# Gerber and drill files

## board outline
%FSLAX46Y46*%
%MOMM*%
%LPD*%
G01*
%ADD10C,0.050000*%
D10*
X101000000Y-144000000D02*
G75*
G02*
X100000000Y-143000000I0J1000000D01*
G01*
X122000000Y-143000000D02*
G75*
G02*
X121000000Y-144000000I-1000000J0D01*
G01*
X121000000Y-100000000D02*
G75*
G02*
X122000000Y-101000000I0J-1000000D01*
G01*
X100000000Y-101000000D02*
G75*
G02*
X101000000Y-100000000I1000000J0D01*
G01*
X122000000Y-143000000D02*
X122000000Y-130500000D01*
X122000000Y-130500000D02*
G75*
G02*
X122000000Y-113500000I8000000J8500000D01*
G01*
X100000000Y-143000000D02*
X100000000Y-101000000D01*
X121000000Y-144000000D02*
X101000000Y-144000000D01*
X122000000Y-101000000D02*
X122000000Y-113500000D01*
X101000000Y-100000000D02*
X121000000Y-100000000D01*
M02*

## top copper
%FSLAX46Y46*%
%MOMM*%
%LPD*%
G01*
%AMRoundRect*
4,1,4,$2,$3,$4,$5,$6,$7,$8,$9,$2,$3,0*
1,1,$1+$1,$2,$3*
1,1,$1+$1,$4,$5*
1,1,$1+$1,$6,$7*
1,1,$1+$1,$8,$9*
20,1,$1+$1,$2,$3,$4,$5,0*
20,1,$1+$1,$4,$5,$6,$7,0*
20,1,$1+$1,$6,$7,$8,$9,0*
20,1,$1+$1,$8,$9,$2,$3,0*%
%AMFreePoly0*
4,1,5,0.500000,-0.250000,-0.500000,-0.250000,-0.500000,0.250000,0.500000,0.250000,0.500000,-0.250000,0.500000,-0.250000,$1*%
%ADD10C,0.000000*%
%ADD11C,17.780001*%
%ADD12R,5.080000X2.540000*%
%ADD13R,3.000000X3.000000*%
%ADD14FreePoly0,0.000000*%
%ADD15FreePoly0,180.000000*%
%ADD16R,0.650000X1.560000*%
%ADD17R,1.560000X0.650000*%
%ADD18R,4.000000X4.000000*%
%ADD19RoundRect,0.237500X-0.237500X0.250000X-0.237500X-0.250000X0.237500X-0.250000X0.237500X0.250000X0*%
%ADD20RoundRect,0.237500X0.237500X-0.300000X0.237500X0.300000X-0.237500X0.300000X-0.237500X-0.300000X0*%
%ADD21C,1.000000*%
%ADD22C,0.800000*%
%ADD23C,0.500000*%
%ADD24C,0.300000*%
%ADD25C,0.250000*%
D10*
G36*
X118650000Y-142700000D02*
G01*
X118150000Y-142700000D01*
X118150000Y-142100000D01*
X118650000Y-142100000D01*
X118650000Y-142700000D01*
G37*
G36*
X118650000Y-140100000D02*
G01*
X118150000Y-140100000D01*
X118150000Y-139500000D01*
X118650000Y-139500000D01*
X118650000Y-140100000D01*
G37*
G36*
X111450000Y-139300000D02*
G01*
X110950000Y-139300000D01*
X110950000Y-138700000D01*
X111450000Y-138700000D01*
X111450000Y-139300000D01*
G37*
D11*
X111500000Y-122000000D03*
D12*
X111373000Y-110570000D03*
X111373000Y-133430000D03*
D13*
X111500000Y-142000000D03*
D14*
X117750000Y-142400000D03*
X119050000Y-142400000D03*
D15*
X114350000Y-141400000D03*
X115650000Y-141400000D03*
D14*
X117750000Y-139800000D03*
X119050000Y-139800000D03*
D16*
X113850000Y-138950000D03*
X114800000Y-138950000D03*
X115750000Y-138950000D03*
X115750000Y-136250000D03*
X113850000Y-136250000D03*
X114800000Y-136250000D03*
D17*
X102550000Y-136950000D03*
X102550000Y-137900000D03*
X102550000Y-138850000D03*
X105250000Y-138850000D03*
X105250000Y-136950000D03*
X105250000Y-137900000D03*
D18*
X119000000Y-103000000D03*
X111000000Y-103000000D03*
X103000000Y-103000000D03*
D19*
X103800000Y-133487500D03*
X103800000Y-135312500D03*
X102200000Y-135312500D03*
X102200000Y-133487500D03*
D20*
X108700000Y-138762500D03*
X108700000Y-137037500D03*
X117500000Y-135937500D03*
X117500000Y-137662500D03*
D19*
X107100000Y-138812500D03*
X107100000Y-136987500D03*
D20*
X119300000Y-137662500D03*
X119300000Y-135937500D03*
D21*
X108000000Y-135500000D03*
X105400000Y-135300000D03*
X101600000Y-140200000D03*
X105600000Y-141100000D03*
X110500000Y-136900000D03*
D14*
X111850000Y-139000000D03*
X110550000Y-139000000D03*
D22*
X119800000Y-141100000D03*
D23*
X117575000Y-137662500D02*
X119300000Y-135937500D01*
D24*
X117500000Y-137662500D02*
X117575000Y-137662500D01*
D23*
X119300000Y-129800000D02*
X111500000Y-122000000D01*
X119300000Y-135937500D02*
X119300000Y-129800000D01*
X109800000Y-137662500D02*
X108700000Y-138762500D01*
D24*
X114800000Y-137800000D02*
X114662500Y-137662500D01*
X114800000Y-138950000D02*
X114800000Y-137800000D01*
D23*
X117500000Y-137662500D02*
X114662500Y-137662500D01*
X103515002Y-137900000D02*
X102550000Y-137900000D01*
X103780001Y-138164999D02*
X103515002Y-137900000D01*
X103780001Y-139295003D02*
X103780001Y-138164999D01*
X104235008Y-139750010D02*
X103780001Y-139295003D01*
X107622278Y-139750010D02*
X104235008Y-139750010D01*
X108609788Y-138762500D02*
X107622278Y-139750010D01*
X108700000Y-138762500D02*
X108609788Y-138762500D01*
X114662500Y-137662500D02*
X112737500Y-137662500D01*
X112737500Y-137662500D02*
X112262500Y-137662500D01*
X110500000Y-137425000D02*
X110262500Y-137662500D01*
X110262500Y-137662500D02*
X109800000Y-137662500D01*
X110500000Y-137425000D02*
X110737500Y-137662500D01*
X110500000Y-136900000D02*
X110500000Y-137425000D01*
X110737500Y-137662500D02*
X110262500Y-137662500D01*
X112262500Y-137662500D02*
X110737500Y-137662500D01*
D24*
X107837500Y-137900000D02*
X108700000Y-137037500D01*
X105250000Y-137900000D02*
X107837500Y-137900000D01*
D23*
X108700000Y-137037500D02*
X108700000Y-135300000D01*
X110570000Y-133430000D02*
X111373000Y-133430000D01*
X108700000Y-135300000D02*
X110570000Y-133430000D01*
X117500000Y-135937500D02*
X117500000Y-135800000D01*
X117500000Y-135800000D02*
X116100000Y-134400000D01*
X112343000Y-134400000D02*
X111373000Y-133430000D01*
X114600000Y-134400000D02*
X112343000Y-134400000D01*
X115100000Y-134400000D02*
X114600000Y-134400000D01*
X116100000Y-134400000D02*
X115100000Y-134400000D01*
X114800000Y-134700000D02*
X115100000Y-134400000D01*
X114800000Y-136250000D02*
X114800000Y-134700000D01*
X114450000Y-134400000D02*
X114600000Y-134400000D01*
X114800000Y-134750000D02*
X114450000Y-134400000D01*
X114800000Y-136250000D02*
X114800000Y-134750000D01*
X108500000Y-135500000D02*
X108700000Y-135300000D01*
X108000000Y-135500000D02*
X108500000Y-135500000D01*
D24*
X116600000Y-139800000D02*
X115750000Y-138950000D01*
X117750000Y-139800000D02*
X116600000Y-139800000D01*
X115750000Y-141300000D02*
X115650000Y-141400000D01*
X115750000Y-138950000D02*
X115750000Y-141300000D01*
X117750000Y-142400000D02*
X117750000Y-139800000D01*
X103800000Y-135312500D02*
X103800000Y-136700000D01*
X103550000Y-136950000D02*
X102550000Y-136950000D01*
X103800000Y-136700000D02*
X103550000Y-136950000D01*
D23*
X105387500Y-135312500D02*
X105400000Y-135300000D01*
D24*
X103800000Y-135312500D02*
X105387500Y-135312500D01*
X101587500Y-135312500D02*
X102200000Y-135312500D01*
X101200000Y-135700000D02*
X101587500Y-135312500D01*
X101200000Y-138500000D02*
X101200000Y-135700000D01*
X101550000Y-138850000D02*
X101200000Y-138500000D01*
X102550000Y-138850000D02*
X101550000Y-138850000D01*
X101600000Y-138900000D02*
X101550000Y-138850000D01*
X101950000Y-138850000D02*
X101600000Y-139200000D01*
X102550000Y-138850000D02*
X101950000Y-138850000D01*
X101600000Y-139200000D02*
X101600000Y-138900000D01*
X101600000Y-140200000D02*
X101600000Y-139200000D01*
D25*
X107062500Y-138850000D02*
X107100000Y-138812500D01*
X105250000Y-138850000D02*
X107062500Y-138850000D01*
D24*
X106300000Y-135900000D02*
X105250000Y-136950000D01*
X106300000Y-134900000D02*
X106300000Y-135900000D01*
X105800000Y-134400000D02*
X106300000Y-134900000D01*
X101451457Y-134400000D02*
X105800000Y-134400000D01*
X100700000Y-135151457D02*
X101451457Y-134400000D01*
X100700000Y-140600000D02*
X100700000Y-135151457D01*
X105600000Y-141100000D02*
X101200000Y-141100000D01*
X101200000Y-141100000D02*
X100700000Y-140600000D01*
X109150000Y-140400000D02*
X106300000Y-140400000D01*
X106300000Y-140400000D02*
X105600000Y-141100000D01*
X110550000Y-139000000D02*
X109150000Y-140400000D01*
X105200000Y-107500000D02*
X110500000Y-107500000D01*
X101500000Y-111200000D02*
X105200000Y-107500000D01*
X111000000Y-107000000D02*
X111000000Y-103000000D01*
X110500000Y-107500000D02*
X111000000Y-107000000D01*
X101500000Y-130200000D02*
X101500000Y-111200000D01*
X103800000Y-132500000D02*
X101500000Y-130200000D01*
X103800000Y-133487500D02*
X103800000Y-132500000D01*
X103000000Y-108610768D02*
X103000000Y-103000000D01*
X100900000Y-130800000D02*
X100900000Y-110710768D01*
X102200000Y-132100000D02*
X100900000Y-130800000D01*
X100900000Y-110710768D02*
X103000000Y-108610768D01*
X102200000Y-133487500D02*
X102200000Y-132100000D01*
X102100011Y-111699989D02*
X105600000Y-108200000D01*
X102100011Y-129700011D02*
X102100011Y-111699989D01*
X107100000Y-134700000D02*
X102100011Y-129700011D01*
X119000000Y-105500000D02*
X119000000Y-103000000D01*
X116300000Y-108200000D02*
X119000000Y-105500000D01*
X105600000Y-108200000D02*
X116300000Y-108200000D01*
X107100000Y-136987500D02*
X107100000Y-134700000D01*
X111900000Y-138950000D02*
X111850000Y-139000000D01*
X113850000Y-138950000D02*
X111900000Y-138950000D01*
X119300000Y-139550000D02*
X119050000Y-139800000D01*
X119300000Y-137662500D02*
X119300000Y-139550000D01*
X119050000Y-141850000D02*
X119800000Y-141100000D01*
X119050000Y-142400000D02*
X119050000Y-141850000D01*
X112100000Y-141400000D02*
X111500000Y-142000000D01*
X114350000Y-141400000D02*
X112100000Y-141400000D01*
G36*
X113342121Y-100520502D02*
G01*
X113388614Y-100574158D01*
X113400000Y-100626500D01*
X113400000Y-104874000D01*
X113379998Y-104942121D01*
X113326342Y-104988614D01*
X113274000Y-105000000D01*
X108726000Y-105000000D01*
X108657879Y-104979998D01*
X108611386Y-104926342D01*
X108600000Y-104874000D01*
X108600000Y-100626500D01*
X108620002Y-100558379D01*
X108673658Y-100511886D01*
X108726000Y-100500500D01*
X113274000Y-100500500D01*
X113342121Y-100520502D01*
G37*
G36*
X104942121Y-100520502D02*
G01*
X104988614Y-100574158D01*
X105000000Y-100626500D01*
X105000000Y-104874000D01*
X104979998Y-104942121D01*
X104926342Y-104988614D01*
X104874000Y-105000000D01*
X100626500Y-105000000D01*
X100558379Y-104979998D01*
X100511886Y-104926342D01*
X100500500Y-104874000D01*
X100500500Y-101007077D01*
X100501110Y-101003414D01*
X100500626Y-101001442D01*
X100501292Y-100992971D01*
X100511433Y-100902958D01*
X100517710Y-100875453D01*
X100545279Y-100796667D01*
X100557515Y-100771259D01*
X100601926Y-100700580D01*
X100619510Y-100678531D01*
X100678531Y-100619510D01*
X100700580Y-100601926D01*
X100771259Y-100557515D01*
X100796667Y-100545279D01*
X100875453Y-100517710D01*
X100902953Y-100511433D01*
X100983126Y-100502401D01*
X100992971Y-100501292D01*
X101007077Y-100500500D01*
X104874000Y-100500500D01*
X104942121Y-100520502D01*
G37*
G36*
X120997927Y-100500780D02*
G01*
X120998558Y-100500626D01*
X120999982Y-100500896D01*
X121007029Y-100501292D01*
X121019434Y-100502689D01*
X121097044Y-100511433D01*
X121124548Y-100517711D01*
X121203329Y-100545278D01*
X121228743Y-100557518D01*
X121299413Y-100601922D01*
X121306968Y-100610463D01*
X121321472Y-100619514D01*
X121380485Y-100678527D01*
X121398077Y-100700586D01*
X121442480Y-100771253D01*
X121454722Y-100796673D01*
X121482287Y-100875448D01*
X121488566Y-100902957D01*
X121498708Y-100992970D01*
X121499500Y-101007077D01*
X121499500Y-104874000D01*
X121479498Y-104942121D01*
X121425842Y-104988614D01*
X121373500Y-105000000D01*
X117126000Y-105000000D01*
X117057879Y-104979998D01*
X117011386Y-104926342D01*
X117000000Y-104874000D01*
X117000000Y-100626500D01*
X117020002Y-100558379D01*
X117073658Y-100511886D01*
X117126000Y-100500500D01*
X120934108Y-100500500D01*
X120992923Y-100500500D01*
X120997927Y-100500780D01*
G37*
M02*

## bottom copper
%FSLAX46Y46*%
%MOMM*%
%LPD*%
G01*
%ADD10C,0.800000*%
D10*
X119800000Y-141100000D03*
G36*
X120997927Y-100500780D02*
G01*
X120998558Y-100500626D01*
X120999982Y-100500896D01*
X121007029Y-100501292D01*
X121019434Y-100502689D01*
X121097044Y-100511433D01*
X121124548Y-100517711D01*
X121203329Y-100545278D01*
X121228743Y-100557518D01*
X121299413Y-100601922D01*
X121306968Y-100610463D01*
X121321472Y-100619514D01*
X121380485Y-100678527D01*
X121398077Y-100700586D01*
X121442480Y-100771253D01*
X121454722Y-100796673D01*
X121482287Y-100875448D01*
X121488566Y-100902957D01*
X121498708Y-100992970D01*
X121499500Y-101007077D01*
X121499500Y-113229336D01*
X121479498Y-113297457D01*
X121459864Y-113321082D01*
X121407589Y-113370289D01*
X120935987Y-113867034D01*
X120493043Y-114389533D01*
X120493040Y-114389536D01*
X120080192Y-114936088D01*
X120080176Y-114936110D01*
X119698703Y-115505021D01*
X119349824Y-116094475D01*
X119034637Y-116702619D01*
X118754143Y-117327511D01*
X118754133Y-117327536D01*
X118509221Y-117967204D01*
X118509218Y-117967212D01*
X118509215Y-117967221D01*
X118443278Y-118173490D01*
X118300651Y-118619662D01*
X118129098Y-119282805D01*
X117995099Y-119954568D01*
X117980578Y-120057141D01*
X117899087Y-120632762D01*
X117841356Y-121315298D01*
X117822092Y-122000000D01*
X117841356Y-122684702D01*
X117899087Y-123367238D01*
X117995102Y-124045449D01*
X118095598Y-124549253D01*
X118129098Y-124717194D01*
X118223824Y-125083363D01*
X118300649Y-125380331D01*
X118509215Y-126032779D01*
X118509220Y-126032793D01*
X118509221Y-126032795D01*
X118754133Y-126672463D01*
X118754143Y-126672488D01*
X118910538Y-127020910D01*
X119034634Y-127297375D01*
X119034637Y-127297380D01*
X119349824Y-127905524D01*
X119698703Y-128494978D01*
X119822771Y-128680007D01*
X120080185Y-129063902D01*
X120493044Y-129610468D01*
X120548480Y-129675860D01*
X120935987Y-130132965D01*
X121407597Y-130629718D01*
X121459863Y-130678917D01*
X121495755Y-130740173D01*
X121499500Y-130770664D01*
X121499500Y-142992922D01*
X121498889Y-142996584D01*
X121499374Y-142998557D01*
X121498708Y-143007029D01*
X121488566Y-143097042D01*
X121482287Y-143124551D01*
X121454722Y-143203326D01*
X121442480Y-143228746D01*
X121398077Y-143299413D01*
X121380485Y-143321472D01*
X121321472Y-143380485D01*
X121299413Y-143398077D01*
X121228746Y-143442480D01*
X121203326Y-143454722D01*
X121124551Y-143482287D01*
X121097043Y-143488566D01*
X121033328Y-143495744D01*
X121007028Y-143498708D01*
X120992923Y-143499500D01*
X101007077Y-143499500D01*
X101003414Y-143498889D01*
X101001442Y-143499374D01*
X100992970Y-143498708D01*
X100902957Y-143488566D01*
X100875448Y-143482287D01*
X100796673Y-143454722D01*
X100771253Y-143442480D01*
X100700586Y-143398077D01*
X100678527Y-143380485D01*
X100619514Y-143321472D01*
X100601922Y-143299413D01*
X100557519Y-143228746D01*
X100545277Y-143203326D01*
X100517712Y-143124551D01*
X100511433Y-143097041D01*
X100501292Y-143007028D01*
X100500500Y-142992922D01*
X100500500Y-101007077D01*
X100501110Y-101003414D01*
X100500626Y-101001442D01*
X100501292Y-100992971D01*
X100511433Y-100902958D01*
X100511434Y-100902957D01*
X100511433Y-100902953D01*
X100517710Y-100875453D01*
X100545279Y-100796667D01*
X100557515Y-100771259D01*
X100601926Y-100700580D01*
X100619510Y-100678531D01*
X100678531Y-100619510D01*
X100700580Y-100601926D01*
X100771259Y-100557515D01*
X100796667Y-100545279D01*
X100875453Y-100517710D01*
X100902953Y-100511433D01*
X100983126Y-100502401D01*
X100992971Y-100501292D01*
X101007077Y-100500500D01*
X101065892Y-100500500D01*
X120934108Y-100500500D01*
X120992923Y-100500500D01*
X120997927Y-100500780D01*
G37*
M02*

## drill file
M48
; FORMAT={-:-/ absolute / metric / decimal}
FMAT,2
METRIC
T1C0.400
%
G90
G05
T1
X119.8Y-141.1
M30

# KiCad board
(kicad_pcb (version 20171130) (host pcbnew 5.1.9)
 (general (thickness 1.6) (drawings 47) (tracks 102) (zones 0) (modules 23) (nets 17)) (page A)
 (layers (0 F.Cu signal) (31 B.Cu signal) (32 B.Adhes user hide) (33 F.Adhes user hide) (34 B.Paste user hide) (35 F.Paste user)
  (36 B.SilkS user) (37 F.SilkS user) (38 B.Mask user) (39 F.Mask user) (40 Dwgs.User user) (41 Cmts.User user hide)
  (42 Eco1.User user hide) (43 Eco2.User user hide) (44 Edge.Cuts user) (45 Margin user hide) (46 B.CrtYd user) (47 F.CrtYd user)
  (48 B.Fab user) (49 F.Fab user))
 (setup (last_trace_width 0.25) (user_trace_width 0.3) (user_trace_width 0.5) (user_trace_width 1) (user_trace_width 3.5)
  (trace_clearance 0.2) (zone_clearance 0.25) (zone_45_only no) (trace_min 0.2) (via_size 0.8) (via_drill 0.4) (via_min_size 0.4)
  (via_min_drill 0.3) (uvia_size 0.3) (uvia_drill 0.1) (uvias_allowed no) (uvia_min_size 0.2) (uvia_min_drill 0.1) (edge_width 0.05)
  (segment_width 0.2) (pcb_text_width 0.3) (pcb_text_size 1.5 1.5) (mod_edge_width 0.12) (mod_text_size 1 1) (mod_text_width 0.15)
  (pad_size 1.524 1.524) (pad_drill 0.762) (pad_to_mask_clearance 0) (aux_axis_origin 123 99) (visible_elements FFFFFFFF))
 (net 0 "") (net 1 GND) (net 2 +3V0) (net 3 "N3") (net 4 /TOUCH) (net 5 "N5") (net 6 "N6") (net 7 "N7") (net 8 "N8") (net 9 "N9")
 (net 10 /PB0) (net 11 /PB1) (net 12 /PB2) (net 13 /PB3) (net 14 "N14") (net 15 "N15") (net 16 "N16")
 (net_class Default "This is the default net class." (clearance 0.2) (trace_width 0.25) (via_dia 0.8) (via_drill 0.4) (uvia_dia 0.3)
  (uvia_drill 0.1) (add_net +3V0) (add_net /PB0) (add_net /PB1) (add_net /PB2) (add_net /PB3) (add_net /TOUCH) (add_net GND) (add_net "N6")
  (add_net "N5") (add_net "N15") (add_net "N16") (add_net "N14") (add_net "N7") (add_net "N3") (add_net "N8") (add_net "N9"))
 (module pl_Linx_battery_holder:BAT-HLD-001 (layer F.Cu) (at 111.5 122 90)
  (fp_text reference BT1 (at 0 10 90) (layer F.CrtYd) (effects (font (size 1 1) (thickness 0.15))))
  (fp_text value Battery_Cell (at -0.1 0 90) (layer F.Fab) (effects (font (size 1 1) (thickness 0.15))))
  (pad 2 smd circle (at 0 0 90) (size 17.780001 17.780001) (layers F.Cu F.Mask) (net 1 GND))
  (pad 3 smd rect (at 11.43 -0.127 90) (size 2.54 5.08) (layers F.Cu F.Paste F.Mask))
  (pad 1 smd rect (at -11.43 -0.127 90) (size 2.54 5.08) (layers F.Cu F.Paste F.Mask) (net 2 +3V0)))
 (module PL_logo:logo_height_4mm (layer F.Cu) (at 118.5 111.5)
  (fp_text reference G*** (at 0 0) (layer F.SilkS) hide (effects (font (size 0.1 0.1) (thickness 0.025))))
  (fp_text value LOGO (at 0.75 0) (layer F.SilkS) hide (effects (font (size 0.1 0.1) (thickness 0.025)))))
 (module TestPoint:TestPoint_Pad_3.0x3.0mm (layer F.Cu) (at 111.5 142)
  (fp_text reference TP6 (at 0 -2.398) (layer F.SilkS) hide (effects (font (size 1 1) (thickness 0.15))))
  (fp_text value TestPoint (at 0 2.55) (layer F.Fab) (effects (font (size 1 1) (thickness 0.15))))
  (pad 1 smd rect (at 0 0) (size 3 3) (layers F.Cu F.Mask) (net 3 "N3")))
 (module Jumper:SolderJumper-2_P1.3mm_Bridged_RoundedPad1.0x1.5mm (layer F.Cu) (at 118.4 142.4)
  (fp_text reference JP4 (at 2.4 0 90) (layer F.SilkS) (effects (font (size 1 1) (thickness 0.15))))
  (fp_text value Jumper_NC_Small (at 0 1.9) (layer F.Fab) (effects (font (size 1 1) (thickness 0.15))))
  (fp_poly (pts (xy 0.25 -0.3) (xy -0.25 -0.3) (xy -0.25 0.3) (xy 0.25 0.3)) (layer F.Cu) (width 0))
  (pad 1 smd custom (at -0.65 0) (size 1 0.5) (layers F.Cu F.Mask) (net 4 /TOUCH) (zone_connect 2)
   (options (clearance outline) (anchor rect)) (primitives))
  (pad 2 smd custom (at 0.65 0) (size 1 0.5) (layers F.Cu F.Mask) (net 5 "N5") (zone_connect 2) (options (clearance outline) (anchor rect))
   (primitives)))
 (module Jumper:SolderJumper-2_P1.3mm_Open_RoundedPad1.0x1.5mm (layer F.Cu) (at 115 141.4 180)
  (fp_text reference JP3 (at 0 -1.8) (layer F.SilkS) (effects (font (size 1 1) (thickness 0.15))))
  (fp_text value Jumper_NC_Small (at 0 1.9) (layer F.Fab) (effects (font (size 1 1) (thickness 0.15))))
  (pad 2 smd custom (at 0.65 0 180) (size 1 0.5) (layers F.Cu F.Mask) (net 3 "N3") (zone_connect 2)
   (options (clearance outline) (anchor rect)) (primitives))
  (pad 1 smd custom (at -0.65 0 180) (size 1 0.5) (layers F.Cu F.Mask) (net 4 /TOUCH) (zone_connect 2)
   (options (clearance outline) (anchor rect)) (primitives)))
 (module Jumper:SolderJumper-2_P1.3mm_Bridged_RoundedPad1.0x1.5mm (layer F.Cu) (at 118.4 139.8)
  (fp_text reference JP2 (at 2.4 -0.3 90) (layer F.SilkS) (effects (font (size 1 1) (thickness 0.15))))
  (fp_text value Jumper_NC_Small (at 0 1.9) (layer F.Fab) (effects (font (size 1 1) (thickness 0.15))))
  (fp_poly (pts (xy 0.25 -0.3) (xy -0.25 -0.3) (xy -0.25 0.3) (xy 0.25 0.3)) (layer F.Cu) (width 0))
  (pad 1 smd custom (at -0.65 0) (size 1 0.5) (layers F.Cu F.Mask) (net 4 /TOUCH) (zone_connect 2)
   (options (clearance outline) (anchor rect)) (primitives))
  (pad 2 smd custom (at 0.65 0) (size 1 0.5) (layers F.Cu F.Mask) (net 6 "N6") (zone_connect 2) (options (clearance outline) (anchor rect))
   (primitives)))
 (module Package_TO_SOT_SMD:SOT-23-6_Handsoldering (layer F.Cu) (at 114.8 137.6 90)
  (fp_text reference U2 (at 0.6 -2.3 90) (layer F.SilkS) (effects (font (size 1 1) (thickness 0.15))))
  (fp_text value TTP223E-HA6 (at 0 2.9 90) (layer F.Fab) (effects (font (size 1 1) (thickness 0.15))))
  (pad 1 smd rect (at -1.35 -0.95 90) (size 1.56 0.65) (layers F.Cu F.Paste F.Mask) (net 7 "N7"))
  (pad 2 smd rect (at -1.35 0 90) (size 1.56 0.65) (layers F.Cu F.Paste F.Mask) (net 1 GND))
  (pad 3 smd rect (at -1.35 0.95 90) (size 1.56 0.65) (layers F.Cu F.Paste F.Mask) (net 4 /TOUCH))
  (pad 4 smd rect (at 1.35 0.95 90) (size 1.56 0.65) (layers F.Cu F.Paste F.Mask) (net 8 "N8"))
  (pad 6 smd rect (at 1.35 -0.95 90) (size 1.56 0.65) (layers F.Cu F.Paste F.Mask) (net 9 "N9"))
  (pad 5 smd rect (at 1.35 0 90) (size 1.56 0.65) (layers F.Cu F.Paste F.Mask) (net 2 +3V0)))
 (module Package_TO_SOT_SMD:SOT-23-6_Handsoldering (layer F.Cu) (at 103.9 137.9)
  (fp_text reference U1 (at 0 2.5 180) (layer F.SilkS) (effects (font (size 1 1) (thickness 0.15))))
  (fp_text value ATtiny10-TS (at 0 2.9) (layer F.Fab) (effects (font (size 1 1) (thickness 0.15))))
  (pad 1 smd rect (at -1.35 -0.95) (size 1.56 0.65) (layers F.Cu F.Paste F.Mask) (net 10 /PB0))
  (pad 2 smd rect (at -1.35 0) (size 1.56 0.65) (layers F.Cu F.Paste F.Mask) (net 1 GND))
  (pad 3 smd rect (at -1.35 0.95) (size 1.56 0.65) (layers F.Cu F.Paste F.Mask) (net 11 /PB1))
  (pad 4 smd rect (at 1.35 0.95) (size 1.56 0.65) (layers F.Cu F.Paste F.Mask) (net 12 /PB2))
  (pad 6 smd rect (at 1.35 -0.95) (size 1.56 0.65) (layers F.Cu F.Paste F.Mask) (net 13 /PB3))
  (pad 5 smd rect (at 1.35 0) (size 1.56 0.65) (layers F.Cu F.Paste F.Mask) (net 2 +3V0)))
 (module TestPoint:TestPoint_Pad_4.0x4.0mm (layer F.Cu) (at 119 103)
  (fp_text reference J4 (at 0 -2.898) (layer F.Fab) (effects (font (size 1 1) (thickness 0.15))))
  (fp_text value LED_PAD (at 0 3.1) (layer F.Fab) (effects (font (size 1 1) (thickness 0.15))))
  (pad 1 smd rect (at 0 0) (size 4 4) (layers F.Cu F.Mask) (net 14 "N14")))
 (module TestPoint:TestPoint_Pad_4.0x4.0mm (layer F.Cu) (at 111 103)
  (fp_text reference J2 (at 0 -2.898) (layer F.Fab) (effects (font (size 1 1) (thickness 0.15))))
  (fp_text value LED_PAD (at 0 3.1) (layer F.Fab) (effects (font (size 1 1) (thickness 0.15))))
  (pad 1 smd rect (at 0 0) (size 4 4) (layers F.Cu F.Mask) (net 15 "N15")))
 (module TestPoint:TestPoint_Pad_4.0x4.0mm (layer F.Cu) (at 103 103)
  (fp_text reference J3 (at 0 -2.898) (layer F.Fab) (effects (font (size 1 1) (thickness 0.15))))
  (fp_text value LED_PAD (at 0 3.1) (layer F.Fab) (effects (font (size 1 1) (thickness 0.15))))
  (pad 1 smd rect (at 0 0) (size 4 4) (layers F.Cu F.Mask) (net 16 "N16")))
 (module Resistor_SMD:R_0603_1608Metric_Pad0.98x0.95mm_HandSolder (layer F.Cu) (at 103.8 134.4 270)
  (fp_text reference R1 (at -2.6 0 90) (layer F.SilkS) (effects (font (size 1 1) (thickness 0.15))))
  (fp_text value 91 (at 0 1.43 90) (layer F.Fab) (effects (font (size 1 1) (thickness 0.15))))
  (pad 1 smd roundrect (at -0.9125 0 270) (size 0.975 0.95) (layers F.Cu F.Paste F.Mask) (roundrect_rratio 0.25) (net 15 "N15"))
  (pad 2 smd roundrect (at 0.9125 0 270) (size 0.975 0.95) (layers F.Cu F.Paste F.Mask) (roundrect_rratio 0.25) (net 10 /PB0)))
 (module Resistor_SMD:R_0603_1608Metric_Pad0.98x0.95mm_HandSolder (layer F.Cu) (at 102.2 134.4 270)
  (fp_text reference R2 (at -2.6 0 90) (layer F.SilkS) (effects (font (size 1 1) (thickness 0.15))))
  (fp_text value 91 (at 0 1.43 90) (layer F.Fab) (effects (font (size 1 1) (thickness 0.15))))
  (pad 2 smd roundrect (at 0.9125 0 270) (size 0.975 0.95) (layers F.Cu F.Paste F.Mask) (roundrect_rratio 0.25) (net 11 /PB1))
  (pad 1 smd roundrect (at -0.9125 0 270) (size 0.975 0.95) (layers F.Cu F.Paste F.Mask) (roundrect_rratio 0.25) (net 16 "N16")))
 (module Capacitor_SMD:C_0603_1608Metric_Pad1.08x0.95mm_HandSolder (layer F.Cu) (at 108.7 137.9 90)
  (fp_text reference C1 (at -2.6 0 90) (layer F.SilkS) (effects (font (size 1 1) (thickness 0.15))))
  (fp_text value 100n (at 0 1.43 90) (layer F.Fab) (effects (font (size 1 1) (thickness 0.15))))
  (pad 1 smd roundrect (at -0.8625 0 90) (size 1.075 0.95) (layers F.Cu F.Paste F.Mask) (roundrect_rratio 0.25) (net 1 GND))
  (pad 2 smd roundrect (at 0.8625 0 90) (size 1.075 0.95) (layers F.Cu F.Paste F.Mask) (roundrect_rratio 0.25) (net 2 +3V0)))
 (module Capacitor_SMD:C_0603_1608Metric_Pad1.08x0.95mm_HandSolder (layer F.Cu) (at 117.5 136.8 90)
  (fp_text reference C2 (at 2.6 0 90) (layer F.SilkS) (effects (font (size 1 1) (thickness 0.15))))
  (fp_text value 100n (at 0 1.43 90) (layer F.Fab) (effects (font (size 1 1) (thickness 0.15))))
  (pad 2 smd roundrect (at 0.8625 0 90) (size 1.075 0.95) (layers F.Cu F.Paste F.Mask) (roundrect_rratio 0.25) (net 2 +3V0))
  (pad 1 smd roundrect (at -0.8625 0 90) (size 1.075 0.95) (layers F.Cu F.Paste F.Mask) (roundrect_rratio 0.25) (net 1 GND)))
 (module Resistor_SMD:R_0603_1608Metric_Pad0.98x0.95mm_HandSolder (layer F.Cu) (at 107.1 137.9 270)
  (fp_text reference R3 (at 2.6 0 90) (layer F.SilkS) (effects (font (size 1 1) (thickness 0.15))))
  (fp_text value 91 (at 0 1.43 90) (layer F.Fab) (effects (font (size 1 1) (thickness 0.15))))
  (pad 2 smd roundrect (at 0.9125 0 270) (size 0.975 0.95) (layers F.Cu F.Paste F.Mask) (roundrect_rratio 0.25) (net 12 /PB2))
  (pad 1 smd roundrect (at -0.9125 0 270) (size 0.975 0.95) (layers F.Cu F.Paste F.Mask) (roundrect_rratio 0.25) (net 14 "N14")))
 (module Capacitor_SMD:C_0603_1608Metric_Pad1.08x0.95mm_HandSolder (layer F.Cu) (at 119.3 136.8 90)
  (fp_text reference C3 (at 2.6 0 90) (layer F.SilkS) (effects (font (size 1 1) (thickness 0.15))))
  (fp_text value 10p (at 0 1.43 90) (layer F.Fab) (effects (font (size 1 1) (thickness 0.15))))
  (pad 1 smd roundrect (at -0.8625 0 90) (size 1.075 0.95) (layers F.Cu F.Paste F.Mask) (roundrect_rratio 0.25) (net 6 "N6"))
  (pad 2 smd roundrect (at 0.8625 0 90) (size 1.075 0.95) (layers F.Cu F.Paste F.Mask) (roundrect_rratio 0.25) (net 1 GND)))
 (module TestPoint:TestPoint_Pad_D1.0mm (layer F.Cu) (at 108 135.5)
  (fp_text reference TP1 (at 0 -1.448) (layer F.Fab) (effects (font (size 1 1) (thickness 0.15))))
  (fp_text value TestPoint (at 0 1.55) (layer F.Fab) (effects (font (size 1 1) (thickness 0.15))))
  (pad 1 smd circle (at 0 0) (size 1 1) (layers F.Cu F.Mask) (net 2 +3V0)))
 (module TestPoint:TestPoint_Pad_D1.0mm (layer F.Cu) (at 105.4 135.3)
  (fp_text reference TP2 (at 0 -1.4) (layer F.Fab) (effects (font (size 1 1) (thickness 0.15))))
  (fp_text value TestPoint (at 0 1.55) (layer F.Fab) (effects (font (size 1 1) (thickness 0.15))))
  (pad 1 smd circle (at 0 0) (size 1 1) (layers F.Cu F.Mask) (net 10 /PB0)))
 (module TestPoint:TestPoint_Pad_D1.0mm (layer F.Cu) (at 101.6 140.2)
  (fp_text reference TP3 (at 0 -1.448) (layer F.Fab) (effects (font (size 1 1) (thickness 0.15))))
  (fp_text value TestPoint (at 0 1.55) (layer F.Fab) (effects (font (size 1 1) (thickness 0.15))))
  (pad 1 smd circle (at 0 0) (size 1 1) (layers F.Cu F.Mask) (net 11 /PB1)))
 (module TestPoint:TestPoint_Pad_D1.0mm (layer F.Cu) (at 105.6 141.1)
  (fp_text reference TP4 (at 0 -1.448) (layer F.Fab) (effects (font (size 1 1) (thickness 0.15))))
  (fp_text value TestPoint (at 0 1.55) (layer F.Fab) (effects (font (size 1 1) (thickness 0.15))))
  (pad 1 smd circle (at 0 0) (size 1 1) (layers F.Cu F.Mask) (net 13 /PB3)))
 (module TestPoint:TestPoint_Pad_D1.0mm (layer F.Cu) (at 110.5 136.9)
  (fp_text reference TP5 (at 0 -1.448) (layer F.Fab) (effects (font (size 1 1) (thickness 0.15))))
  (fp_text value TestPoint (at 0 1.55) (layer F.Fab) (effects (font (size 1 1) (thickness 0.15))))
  (pad 1 smd circle (at 0 0) (size 1 1) (layers F.Cu F.Mask) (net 1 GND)))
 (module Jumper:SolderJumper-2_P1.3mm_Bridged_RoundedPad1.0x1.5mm (layer F.Cu) (at 111.2 139)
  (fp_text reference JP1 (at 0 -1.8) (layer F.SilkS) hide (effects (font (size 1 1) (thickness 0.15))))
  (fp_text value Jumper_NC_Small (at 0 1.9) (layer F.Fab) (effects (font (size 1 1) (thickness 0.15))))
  (fp_poly (pts (xy 0.25 -0.3) (xy -0.25 -0.3) (xy -0.25 0.3) (xy 0.25 0.3)) (layer F.Cu) (width 0))
  (pad 2 smd custom (at 0.65 0) (size 1 0.5) (layers F.Cu F.Mask) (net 7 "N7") (zone_connect 2) (options (clearance outline) (anchor rect))
   (primitives))
  (pad 1 smd custom (at -0.65 0) (size 1 0.5) (layers F.Cu F.Mask) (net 13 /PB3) (zone_connect 2)
   (options (clearance outline) (anchor rect)) (primitives)))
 (gr_arc (start 101 143) (end 100 143) (angle -90) (layer Edge.Cuts) (width 0.05))
 (gr_arc (start 121 143) (end 121 144) (angle -90) (layer Edge.Cuts) (width 0.05))
 (gr_arc (start 121 101) (end 122 101) (angle -90) (layer Edge.Cuts) (width 0.05))
 (gr_arc (start 101 101) (end 101 100) (angle -90) (layer Edge.Cuts) (width 0.05))
 (gr_line (start 122 143) (end 122 130.5) (layer Edge.Cuts) (width 0.05))
 (gr_arc (start 130 122) (end 122 113.5) (angle -93.47140918) (layer Edge.Cuts) (width 0.05))
 (gr_line (start 100 143) (end 100 101) (layer Edge.Cuts) (width 0.05))
 (gr_line (start 121 144) (end 101 144) (layer Edge.Cuts) (width 0.05))
 (gr_line (start 122 101) (end 122 113.5) (layer Edge.Cuts) (width 0.05))
 (gr_line (start 101 100) (end 121 100) (layer Edge.Cuts) (width 0.05))
 (segment (start 117.575 137.6625) (end 119.3 135.9375) (width 0.5) (layer F.Cu) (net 1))
 (segment (start 117.5 137.6625) (end 117.575 137.6625) (width 0.3) (layer F.Cu) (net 1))
 (segment (start 119.3 129.8) (end 111.5 122) (width 0.5) (layer F.Cu) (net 1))
 (segment (start 119.3 135.9375) (end 119.3 129.8) (width 0.5) (layer F.Cu) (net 1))
 (segment (start 109.8 137.6625) (end 108.7 138.7625) (width 0.5) (layer F.Cu) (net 1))
 (segment (start 114.8 137.8) (end 114.6625 137.6625) (width 0.3) (layer F.Cu) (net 1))
 (segment (start 114.8 138.95) (end 114.8 137.8) (width 0.3) (layer F.Cu) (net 1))
 (segment (start 117.5 137.6625) (end 114.6625 137.6625) (width 0.5) (layer F.Cu) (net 1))
 (segment (start 103.515002 137.9) (end 102.55 137.9) (width 0.5) (layer F.Cu) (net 1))
 (segment (start 103.780001 138.164999) (end 103.515002 137.9) (width 0.5) (layer F.Cu) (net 1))
 (segment (start 103.780001 139.295003) (end 103.780001 138.164999) (width 0.5) (layer F.Cu) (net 1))
 (segment (start 104.235008 139.75001) (end 103.780001 139.295003) (width 0.5) (layer F.Cu) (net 1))
 (segment (start 107.622278 139.75001) (end 104.235008 139.75001) (width 0.5) (layer F.Cu) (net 1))
 (segment (start 108.609788 138.7625) (end 107.622278 139.75001) (width 0.5) (layer F.Cu) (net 1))
 (segment (start 108.7 138.7625) (end 108.609788 138.7625) (width 0.5) (layer F.Cu) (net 1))
 (segment (start 114.6625 137.6625) (end 112.7375 137.6625) (width 0.5) (layer F.Cu) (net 1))
 (segment (start 112.7375 137.6625) (end 112.2625 137.6625) (width 0.5) (layer F.Cu) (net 1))
 (segment (start 110.5 137.425) (end 110.2625 137.6625) (width 0.5) (layer F.Cu) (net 1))
 (segment (start 110.2625 137.6625) (end 109.8 137.6625) (width 0.5) (layer F.Cu) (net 1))
 (segment (start 110.5 137.425) (end 110.7375 137.6625) (width 0.5) (layer F.Cu) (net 1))
 (segment (start 110.5 136.9) (end 110.5 137.425) (width 0.5) (layer F.Cu) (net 1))
 (segment (start 110.7375 137.6625) (end 110.2625 137.6625) (width 0.5) (layer F.Cu) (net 1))
 (segment (start 112.2625 137.6625) (end 110.7375 137.6625) (width 0.5) (layer F.Cu) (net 1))
 (segment (start 107.8375 137.9) (end 108.7 137.0375) (width 0.3) (layer F.Cu) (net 2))
 (segment (start 105.25 137.9) (end 107.8375 137.9) (width 0.3) (layer F.Cu) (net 2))
 (segment (start 108.7 137.0375) (end 108.7 135.3) (width 0.5) (layer F.Cu) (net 2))
 (segment (start 110.57 133.43) (end 111.373 133.43) (width 0.5) (layer F.Cu) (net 2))
 (segment (start 108.7 135.3) (end 110.57 133.43) (width 0.5) (layer F.Cu) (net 2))
 (segment (start 117.5 135.9375) (end 117.5 135.8) (width 0.5) (layer F.Cu) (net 2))
 (segment (start 117.5 135.8) (end 116.1 134.4) (width 0.5) (layer F.Cu) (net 2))
 (segment (start 112.343 134.4) (end 111.373 133.43) (width 0.5) (layer F.Cu) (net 2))
 (segment (start 114.6 134.4) (end 112.343 134.4) (width 0.5) (layer F.Cu) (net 2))
 (segment (start 115.1 134.4) (end 114.6 134.4) (width 0.5) (layer F.Cu) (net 2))
 (segment (start 116.1 134.4) (end 115.1 134.4) (width 0.5) (layer F.Cu) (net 2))
 (segment (start 114.8 134.7) (end 115.1 134.4) (width 0.5) (layer F.Cu) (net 2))
 (segment (start 114.8 136.25) (end 114.8 134.7) (width 0.5) (layer F.Cu) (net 2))
 (segment (start 114.45 134.4) (end 114.6 134.4) (width 0.5) (layer F.Cu) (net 2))
 (segment (start 114.8 134.75) (end 114.45 134.4) (width 0.5) (layer F.Cu) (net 2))
 (segment (start 114.8 136.25) (end 114.8 134.75) (width 0.5) (layer F.Cu) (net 2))
 (segment (start 108.5 135.5) (end 108.7 135.3) (width 0.5) (layer F.Cu) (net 2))
 (segment (start 108 135.5) (end 108.5 135.5) (width 0.5) (layer F.Cu) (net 2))
 (segment (start 116.6 139.8) (end 115.75 138.95) (width 0.3) (layer F.Cu) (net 4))
 (segment (start 117.75 139.8) (end 116.6 139.8) (width 0.3) (layer F.Cu) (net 4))
 (segment (start 115.75 141.3) (end 115.65 141.4) (width 0.3) (layer F.Cu) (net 4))
 (segment (start 115.75 138.95) (end 115.75 141.3) (width 0.3) (layer F.Cu) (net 4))
 (segment (start 117.75 142.4) (end 117.75 139.8) (width 0.3) (layer F.Cu) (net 4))
 (segment (start 103.8 135.3125) (end 103.8 136.7) (width 0.3) (layer F.Cu) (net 10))
 (segment (start 103.55 136.95) (end 102.55 136.95) (width 0.3) (layer F.Cu) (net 10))
 (segment (start 103.8 136.7) (end 103.55 136.95) (width 0.3) (layer F.Cu) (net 10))
 (segment (start 105.3875 135.3125) (end 105.4 135.3) (width 0.5) (layer F.Cu) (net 10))
 (segment (start 103.8 135.3125) (end 105.3875 135.3125) (width 0.3) (layer F.Cu) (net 10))
 (segment (start 101.5875 135.3125) (end 102.2 135.3125) (width 0.3) (layer F.Cu) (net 11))
 (segment (start 101.2 135.7) (end 101.5875 135.3125) (width 0.3) (layer F.Cu) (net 11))
 (segment (start 101.2 138.5) (end 101.2 135.7) (width 0.3) (layer F.Cu) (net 11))
 (segment (start 101.55 138.85) (end 101.2 138.5) (width 0.3) (layer F.Cu) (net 11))
 (segment (start 102.55 138.85) (end 101.55 138.85) (width 0.3) (layer F.Cu) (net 11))
 (segment (start 101.6 138.9) (end 101.55 138.85) (width 0.3) (layer F.Cu) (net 11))
 (segment (start 101.95 138.85) (end 101.6 139.2) (width 0.3) (layer F.Cu) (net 11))
 (segment (start 102.55 138.85) (end 101.95 138.85) (width 0.3) (layer F.Cu) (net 11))
 (segment (start 101.6 139.2) (end 101.6 138.9) (width 0.3) (layer F.Cu) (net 11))
 (segment (start 101.6 140.2) (end 101.6 139.2) (width 0.3) (layer F.Cu) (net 11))
 (segment (start 107.0625 138.85) (end 107.1 138.8125) (width 0.25) (layer F.Cu) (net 12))
 (segment (start 105.25 138.85) (end 107.0625 138.85) (width 0.25) (layer F.Cu) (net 12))
 (segment (start 106.3 135.9) (end 105.25 136.95) (width 0.3) (layer F.Cu) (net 13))
 (segment (start 106.3 134.9) (end 106.3 135.9) (width 0.3) (layer F.Cu) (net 13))
 (segment (start 105.8 134.4) (end 106.3 134.9) (width 0.3) (layer F.Cu) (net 13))
 (segment (start 101.451457 134.4) (end 105.8 134.4) (width 0.3) (layer F.Cu) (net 13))
 (segment (start 100.7 135.151457) (end 101.451457 134.4) (width 0.3) (layer F.Cu) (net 13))
 (segment (start 100.7 140.6) (end 100.7 135.151457) (width 0.3) (layer F.Cu) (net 13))
 (segment (start 105.6 141.1) (end 101.2 141.1) (width 0.3) (layer F.Cu) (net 13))
 (segment (start 101.2 141.1) (end 100.7 140.6) (width 0.3) (layer F.Cu) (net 13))
 (segment (start 109.15 140.4) (end 106.3 140.4) (width 0.3) (layer F.Cu) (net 13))
 (segment (start 106.3 140.4) (end 105.6 141.1) (width 0.3) (layer F.Cu) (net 13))
 (segment (start 110.55 139) (end 109.15 140.4) (width 0.3) (layer F.Cu) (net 13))
 (segment (start 105.2 107.5) (end 110.5 107.5) (width 0.3) (layer F.Cu) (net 15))
 (segment (start 101.5 111.2) (end 105.2 107.5) (width 0.3) (layer F.Cu) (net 15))
 (segment (start 111 107) (end 111 103) (width 0.3) (layer F.Cu) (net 15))
 (segment (start 110.5 107.5) (end 111 107) (width 0.3) (layer F.Cu) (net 15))
 (segment (start 101.5 130.2) (end 101.5 111.2) (width 0.3) (layer F.Cu) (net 15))
 (segment (start 103.8 132.5) (end 101.5 130.2) (width 0.3) (layer F.Cu) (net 15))
 (segment (start 103.8 133.4875) (end 103.8 132.5) (width 0.3) (layer F.Cu) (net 15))
 (segment (start 103 108.610768) (end 103 103) (width 0.3) (layer F.Cu) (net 16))
 (segment (start 100.9 130.8) (end 100.9 110.710768) (width 0.3) (layer F.Cu) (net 16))
 (segment (start 102.2 132.1) (end 100.9 130.8) (width 0.3) (layer F.Cu) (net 16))
 (segment (start 100.9 110.710768) (end 103 108.610768) (width 0.3) (layer F.Cu) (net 16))
 (segment (start 102.2 133.4875) (end 102.2 132.1) (width 0.3) (layer F.Cu) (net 16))
 (segment (start 102.100011 111.699989) (end 105.6 108.2) (width 0.3) (layer F.Cu) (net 14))
 (segment (start 102.100011 129.700011) (end 102.100011 111.699989) (width 0.3) (layer F.Cu) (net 14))
 (segment (start 107.1 134.7) (end 102.100011 129.700011) (width 0.3) (layer F.Cu) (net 14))
 (segment (start 119 105.5) (end 119 103) (width 0.3) (layer F.Cu) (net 14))
 (segment (start 116.3 108.2) (end 119 105.5) (width 0.3) (layer F.Cu) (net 14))
 (segment (start 105.6 108.2) (end 116.3 108.2) (width 0.3) (layer F.Cu) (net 14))
 (segment (start 107.1 136.9875) (end 107.1 134.7) (width 0.3) (layer F.Cu) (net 14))
 (segment (start 111.9 138.95) (end 111.85 139) (width 0.3) (layer F.Cu) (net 7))
 (segment (start 113.85 138.95) (end 111.9 138.95) (width 0.3) (layer F.Cu) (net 7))
 (segment (start 119.3 139.55) (end 119.05 139.8) (width 0.3) (layer F.Cu) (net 6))
 (segment (start 119.3 137.6625) (end 119.3 139.55) (width 0.3) (layer F.Cu) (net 6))
 (via (at 119.8 141.1) (size 0.8) (drill 0.4) (layers F.Cu B.Cu) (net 5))
 (segment (start 119.05 141.85) (end 119.8 141.1) (width 0.3) (layer F.Cu) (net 5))
 (segment (start 119.05 142.4) (end 119.05 141.85) (width 0.3) (layer F.Cu) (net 5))
 (segment (start 112.1 141.4) (end 111.5 142) (width 0.3) (layer F.Cu) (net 3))
 (segment (start 114.35 141.4) (end 112.1 141.4) (width 0.3) (layer F.Cu) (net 3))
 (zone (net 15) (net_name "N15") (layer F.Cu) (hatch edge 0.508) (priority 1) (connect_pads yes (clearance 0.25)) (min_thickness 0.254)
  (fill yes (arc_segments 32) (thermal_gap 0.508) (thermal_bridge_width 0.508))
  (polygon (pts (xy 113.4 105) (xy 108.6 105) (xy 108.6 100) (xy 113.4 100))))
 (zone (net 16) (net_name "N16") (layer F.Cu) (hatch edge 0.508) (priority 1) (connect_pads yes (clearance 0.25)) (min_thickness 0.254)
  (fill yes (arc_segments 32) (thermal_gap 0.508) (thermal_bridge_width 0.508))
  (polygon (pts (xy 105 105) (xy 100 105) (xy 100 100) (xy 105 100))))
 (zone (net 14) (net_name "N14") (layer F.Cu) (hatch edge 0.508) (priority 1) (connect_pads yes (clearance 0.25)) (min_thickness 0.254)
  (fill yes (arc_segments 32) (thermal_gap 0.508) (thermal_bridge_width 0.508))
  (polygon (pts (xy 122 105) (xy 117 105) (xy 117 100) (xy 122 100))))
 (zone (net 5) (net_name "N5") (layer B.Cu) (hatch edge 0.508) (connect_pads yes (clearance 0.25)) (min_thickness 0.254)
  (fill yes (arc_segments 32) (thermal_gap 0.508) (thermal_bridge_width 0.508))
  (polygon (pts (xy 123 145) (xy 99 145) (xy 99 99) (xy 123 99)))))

